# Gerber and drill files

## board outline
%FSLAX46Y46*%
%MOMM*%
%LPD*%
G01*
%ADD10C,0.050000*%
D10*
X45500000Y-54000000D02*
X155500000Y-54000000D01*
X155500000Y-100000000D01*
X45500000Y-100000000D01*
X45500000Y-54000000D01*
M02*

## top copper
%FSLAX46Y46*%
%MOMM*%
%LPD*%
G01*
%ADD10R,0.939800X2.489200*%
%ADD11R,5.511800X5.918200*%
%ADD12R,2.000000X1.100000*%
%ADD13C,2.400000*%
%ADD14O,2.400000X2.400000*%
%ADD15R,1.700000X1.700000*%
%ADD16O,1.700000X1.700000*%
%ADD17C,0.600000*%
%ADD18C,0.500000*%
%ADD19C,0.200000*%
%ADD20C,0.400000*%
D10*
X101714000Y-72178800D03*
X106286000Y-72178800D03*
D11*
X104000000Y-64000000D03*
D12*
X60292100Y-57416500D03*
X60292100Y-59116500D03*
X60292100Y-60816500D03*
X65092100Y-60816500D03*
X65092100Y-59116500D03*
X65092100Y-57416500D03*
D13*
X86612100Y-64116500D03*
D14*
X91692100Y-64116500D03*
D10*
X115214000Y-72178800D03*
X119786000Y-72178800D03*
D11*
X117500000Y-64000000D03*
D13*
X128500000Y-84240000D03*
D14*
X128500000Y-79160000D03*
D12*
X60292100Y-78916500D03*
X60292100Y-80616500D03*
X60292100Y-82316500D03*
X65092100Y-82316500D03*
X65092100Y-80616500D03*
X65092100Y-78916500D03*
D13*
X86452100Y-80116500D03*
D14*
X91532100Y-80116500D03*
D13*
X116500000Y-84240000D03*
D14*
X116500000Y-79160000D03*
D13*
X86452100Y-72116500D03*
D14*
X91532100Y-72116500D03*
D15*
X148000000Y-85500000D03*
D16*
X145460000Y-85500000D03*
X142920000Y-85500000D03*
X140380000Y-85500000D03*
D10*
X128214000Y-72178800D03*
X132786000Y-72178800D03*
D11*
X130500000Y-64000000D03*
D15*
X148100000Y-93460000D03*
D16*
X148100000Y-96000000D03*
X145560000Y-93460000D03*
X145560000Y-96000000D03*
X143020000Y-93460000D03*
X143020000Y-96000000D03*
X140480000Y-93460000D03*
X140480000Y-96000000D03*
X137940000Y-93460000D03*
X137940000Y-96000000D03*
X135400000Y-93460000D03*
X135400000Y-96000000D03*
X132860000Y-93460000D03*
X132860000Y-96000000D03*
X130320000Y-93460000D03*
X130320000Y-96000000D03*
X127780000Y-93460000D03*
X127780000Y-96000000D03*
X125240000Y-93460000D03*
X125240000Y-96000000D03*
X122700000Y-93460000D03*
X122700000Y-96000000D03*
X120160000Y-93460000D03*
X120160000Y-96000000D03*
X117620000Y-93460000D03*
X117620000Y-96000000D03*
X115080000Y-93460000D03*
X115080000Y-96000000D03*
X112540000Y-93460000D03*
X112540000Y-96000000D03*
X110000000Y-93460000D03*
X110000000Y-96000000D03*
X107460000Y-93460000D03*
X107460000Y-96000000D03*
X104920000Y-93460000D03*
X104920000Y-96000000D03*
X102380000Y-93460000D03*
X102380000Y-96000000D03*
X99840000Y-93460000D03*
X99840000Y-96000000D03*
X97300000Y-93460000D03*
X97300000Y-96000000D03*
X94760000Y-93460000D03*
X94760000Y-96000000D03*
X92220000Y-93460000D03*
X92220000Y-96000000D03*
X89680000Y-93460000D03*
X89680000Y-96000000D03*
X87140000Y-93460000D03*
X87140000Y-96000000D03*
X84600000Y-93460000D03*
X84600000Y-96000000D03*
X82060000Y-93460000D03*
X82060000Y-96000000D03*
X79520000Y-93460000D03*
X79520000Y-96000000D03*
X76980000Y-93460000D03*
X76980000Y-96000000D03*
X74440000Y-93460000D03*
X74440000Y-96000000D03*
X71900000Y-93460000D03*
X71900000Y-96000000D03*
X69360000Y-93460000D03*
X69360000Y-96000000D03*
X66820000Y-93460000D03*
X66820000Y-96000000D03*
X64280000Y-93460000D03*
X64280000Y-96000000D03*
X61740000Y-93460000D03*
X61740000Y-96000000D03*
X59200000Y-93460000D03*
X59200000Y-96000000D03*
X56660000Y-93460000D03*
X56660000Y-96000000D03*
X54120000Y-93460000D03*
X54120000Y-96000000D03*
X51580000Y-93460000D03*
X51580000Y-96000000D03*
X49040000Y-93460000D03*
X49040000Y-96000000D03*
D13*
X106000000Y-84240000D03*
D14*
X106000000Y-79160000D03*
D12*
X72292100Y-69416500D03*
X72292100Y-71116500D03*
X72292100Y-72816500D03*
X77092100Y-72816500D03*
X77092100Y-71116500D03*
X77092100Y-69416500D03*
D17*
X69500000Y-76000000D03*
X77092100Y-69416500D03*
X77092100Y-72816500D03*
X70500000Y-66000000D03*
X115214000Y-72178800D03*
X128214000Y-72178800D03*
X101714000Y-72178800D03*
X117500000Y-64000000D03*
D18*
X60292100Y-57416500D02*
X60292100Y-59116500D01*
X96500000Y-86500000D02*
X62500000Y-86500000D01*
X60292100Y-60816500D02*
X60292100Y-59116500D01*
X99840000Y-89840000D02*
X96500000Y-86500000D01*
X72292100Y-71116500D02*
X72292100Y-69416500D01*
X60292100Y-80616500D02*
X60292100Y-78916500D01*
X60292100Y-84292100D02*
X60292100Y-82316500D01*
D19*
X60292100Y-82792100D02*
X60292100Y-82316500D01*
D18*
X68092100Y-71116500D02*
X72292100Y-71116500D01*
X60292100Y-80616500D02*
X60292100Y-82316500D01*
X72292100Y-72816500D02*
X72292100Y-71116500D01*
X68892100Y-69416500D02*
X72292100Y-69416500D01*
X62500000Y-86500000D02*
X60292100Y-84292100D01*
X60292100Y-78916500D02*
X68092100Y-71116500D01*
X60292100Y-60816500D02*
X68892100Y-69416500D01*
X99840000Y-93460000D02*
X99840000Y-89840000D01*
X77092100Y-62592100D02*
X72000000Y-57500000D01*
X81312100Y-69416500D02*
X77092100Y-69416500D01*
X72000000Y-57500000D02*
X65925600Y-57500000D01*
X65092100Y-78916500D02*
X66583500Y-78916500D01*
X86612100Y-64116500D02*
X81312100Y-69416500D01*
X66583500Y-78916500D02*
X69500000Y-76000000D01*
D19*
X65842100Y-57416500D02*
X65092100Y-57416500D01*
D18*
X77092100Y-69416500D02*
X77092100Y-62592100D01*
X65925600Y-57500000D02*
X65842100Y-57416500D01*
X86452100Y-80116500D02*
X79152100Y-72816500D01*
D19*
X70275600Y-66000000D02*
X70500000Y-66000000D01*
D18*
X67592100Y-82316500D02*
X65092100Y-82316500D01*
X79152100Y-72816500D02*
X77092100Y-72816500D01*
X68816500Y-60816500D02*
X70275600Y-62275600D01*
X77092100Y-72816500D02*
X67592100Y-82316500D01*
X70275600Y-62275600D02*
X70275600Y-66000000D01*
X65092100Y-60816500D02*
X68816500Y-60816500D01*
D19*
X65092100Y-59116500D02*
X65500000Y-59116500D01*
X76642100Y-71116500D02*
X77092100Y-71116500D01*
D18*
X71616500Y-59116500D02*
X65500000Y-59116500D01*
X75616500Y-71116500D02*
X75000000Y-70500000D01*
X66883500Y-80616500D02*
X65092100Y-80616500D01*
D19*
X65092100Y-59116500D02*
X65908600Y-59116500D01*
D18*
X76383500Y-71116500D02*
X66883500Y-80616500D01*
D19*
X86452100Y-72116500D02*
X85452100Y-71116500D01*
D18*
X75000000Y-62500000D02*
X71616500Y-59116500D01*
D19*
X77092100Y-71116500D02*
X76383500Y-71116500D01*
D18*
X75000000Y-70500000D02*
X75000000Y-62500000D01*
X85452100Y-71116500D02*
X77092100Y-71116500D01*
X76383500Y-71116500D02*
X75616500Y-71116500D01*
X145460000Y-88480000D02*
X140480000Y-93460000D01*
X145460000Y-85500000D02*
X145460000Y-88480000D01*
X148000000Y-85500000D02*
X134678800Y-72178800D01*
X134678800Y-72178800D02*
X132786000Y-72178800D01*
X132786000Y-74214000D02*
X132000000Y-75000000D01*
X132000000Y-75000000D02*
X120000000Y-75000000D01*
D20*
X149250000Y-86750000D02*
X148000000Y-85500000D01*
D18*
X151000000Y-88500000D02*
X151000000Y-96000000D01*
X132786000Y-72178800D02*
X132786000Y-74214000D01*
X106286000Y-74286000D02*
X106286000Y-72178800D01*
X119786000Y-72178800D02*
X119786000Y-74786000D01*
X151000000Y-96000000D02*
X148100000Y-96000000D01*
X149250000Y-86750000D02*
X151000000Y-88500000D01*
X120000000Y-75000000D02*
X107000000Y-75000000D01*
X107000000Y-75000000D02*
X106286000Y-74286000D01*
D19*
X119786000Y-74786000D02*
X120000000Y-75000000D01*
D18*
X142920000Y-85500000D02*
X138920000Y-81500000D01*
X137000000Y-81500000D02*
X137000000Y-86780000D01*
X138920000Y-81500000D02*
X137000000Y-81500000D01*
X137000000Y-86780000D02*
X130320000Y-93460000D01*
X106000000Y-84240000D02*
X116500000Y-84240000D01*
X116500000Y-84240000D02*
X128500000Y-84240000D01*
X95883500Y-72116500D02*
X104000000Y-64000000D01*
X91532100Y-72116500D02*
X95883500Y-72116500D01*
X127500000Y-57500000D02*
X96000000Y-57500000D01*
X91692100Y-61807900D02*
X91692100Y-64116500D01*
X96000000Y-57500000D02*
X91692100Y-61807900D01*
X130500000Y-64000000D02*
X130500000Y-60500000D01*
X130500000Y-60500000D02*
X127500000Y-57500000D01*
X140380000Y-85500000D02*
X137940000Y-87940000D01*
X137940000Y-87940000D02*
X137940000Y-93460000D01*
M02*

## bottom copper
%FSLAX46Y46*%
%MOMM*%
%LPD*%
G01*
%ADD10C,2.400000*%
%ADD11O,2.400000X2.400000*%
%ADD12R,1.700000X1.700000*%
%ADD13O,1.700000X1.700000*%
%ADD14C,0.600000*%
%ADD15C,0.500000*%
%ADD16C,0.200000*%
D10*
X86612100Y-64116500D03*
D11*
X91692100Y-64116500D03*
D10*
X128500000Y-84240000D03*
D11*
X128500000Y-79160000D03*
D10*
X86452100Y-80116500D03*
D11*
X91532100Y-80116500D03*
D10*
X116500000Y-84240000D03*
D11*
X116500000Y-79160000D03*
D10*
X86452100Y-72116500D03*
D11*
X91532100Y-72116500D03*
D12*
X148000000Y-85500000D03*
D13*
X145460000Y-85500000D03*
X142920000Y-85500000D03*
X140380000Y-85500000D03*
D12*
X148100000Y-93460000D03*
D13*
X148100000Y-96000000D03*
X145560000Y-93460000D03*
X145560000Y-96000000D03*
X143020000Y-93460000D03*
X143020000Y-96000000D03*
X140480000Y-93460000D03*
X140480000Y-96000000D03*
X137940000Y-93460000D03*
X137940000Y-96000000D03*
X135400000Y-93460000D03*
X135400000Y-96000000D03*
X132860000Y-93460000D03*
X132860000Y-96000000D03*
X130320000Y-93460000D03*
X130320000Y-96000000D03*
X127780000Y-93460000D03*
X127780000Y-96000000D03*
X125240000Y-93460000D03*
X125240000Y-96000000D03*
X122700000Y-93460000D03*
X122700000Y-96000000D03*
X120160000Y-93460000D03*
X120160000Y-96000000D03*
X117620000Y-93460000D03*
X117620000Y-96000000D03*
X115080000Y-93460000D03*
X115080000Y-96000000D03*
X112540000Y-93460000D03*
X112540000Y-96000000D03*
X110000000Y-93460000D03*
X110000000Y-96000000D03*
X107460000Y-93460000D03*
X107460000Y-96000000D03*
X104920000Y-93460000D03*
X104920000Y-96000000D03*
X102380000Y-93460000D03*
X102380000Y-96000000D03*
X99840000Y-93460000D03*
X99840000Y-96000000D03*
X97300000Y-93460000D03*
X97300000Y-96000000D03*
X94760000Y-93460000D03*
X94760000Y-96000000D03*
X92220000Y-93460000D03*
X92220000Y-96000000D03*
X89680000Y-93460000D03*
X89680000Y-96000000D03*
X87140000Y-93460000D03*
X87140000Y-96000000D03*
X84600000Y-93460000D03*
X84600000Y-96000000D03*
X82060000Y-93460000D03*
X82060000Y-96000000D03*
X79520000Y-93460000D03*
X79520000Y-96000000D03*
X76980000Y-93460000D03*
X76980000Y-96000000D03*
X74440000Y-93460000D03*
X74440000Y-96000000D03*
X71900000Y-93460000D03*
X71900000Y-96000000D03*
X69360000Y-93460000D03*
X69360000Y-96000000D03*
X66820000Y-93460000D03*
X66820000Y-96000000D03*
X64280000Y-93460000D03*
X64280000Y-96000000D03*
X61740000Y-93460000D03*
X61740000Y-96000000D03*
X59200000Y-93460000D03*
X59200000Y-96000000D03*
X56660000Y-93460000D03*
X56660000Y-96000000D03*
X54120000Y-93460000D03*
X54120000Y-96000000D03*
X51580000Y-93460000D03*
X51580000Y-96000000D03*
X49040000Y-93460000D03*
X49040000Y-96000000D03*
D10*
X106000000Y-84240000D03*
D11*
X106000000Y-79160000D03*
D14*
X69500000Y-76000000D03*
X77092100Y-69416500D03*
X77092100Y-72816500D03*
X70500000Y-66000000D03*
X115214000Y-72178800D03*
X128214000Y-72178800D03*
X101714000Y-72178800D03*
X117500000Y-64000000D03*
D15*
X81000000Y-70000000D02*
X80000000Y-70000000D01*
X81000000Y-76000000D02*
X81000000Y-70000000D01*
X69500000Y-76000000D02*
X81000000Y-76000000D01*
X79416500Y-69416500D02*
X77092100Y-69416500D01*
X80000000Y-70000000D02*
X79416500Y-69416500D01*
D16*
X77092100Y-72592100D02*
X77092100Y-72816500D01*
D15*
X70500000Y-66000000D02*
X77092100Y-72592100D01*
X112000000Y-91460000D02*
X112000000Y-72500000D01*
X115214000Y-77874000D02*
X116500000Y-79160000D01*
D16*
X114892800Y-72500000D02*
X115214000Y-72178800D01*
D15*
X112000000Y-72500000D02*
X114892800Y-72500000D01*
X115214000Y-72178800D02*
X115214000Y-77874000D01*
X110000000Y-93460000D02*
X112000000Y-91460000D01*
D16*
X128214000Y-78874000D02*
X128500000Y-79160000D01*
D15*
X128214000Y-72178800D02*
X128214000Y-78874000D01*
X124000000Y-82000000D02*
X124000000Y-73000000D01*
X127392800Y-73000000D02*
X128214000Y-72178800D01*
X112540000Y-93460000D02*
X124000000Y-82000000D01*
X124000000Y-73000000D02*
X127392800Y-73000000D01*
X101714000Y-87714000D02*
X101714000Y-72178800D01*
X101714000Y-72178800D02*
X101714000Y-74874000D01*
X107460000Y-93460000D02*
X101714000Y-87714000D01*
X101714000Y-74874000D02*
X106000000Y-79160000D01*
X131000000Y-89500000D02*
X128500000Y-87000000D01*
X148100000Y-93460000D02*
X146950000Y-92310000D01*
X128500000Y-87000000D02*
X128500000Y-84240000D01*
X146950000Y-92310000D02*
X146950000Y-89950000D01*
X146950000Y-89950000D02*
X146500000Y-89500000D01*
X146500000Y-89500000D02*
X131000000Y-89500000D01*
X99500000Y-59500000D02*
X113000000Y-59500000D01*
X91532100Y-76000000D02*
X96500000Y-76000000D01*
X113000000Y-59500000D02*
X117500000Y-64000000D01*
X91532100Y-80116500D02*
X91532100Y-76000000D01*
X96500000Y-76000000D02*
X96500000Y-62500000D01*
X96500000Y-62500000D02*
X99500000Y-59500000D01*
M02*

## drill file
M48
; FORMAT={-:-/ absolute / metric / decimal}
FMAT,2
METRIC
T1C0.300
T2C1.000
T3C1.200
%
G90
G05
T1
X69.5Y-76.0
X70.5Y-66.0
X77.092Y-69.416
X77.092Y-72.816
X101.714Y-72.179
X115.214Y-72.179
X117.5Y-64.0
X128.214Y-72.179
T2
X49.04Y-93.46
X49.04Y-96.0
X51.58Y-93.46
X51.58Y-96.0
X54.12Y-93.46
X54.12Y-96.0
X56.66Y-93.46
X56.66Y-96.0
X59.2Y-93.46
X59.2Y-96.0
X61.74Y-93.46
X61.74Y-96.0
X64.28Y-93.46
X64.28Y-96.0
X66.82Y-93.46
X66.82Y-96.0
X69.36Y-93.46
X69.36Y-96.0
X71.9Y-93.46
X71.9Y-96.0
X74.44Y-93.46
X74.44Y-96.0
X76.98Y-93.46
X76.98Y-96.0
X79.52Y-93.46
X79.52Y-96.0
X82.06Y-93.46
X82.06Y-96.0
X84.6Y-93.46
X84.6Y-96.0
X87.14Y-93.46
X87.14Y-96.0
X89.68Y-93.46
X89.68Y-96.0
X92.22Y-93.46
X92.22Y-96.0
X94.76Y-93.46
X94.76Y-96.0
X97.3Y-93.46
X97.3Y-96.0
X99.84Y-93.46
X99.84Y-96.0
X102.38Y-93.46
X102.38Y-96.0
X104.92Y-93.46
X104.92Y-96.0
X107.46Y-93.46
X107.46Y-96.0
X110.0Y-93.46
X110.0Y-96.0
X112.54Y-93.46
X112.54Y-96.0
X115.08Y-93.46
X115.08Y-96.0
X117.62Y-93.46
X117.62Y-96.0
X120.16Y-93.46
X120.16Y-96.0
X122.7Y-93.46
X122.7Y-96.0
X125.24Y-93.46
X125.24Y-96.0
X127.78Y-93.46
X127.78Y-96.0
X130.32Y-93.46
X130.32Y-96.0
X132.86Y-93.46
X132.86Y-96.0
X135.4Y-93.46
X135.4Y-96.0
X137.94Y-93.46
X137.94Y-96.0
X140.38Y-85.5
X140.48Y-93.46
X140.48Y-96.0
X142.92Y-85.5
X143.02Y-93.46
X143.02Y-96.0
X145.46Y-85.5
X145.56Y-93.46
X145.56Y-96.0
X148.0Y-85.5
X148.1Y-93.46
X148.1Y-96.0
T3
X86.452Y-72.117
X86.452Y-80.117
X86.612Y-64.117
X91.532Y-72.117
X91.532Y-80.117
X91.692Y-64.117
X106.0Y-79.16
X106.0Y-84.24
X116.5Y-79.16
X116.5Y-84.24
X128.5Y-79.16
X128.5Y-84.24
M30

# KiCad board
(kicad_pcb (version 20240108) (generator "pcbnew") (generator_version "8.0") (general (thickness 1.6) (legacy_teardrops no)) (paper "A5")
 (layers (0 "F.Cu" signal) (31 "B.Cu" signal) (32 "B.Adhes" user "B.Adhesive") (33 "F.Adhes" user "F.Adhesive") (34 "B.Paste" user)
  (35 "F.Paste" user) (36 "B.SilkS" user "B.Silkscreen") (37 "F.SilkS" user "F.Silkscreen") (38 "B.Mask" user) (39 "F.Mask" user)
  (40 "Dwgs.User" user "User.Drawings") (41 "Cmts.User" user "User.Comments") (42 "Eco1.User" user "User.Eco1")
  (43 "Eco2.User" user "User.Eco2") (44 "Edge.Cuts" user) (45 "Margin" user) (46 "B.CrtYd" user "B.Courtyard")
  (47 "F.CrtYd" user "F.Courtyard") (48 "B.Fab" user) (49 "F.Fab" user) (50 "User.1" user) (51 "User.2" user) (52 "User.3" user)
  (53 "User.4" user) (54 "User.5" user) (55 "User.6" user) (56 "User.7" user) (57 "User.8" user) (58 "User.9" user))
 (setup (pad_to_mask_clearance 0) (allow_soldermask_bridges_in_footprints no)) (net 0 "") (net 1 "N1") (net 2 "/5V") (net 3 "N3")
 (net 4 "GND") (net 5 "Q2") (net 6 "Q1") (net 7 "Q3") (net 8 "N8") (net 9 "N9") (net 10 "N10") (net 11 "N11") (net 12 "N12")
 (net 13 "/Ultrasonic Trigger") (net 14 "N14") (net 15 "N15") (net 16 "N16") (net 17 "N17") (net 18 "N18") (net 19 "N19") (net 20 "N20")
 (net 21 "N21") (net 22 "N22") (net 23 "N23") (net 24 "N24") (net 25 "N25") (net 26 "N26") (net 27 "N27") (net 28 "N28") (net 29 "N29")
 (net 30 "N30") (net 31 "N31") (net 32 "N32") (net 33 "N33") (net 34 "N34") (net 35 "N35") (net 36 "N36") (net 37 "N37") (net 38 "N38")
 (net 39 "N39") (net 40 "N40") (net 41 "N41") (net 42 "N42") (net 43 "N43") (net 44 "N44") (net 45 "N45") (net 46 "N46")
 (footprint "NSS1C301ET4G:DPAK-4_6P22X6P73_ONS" (layer "F.Cu") (at 104 65.7653)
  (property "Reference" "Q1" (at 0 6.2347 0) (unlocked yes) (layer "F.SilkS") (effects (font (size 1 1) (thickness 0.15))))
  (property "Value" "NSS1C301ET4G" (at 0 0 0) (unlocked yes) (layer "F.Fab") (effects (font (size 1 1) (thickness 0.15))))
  (pad "1" smd rect (at -2.286 6.4135) (size 0.9398 2.4892) (layers "F.Cu" "F.Paste" "F.Mask") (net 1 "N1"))
  (pad "2" smd rect (at 2.286 6.4135) (size 0.9398 2.4892) (layers "F.Cu" "F.Paste" "F.Mask") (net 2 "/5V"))
  (pad "3" smd rect (at 0 -1.7653) (size 5.5118 5.9182) (layers "F.Cu" "F.Paste" "F.Mask") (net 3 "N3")))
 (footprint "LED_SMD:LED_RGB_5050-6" (layer "F.Cu") (at 62.6921 59.1165)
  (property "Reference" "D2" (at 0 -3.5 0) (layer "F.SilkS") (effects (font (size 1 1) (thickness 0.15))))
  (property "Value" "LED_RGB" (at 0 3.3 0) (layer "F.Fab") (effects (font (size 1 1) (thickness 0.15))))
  (pad "1" smd rect (at -2.4 -1.7 90) (size 1.1 2) (layers "F.Cu" "F.Paste" "F.Mask") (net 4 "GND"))
  (pad "2" smd rect (at -2.4 0 90) (size 1.1 2) (layers "F.Cu" "F.Paste" "F.Mask") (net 4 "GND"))
  (pad "3" smd rect (at -2.4 1.7 90) (size 1.1 2) (layers "F.Cu" "F.Paste" "F.Mask") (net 4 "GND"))
  (pad "4" smd rect (at 2.4 1.7 90) (size 1.1 2) (layers "F.Cu" "F.Paste" "F.Mask") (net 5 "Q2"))
  (pad "5" smd rect (at 2.4 0 90) (size 1.1 2) (layers "F.Cu" "F.Paste" "F.Mask") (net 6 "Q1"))
  (pad "6" smd rect (at 2.4 -1.7 90) (size 1.1 2) (layers "F.Cu" "F.Paste" "F.Mask") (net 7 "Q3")))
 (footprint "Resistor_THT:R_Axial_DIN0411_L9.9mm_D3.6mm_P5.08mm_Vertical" (layer "F.Cu") (at 86.6121 64.1165)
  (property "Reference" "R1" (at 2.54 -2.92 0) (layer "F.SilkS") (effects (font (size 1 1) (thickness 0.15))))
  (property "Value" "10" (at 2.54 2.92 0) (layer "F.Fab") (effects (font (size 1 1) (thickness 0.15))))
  (pad "1" thru_hole circle (at 0 0) (size 2.4 2.4) (drill 1.2) (layers "*.Cu" "*.Mask") (remove_unused_layers no) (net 7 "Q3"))
  (pad "2" thru_hole oval (at 5.08 0) (size 2.4 2.4) (drill 1.2) (layers "*.Cu" "*.Mask") (remove_unused_layers no) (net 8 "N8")))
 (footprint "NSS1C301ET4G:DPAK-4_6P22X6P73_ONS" (layer "F.Cu") (at 117.5 65.7653)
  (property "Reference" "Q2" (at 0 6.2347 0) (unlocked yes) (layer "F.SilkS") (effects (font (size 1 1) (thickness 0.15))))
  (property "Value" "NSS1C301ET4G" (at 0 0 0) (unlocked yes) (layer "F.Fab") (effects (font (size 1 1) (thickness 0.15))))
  (pad "1" smd rect (at -2.286 6.4135) (size 0.9398 2.4892) (layers "F.Cu" "F.Paste" "F.Mask") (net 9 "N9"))
  (pad "2" smd rect (at 2.286 6.4135) (size 0.9398 2.4892) (layers "F.Cu" "F.Paste" "F.Mask") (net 2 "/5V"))
  (pad "3" smd rect (at 0 -1.7653) (size 5.5118 5.9182) (layers "F.Cu" "F.Paste" "F.Mask") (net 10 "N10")))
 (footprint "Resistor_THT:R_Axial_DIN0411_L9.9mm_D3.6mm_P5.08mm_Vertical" (layer "F.Cu") (at 128.5 84.24 90)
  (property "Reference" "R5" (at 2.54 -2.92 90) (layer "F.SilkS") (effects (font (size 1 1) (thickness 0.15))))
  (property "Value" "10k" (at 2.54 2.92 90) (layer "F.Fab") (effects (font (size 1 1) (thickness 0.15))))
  (pad "1" thru_hole circle (at 0 0 90) (size 2.4 2.4) (drill 1.2) (layers "*.Cu" "*.Mask") (remove_unused_layers no) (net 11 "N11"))
  (pad "2" thru_hole oval (at 5.08 0 90) (size 2.4 2.4) (drill 1.2) (layers "*.Cu" "*.Mask") (remove_unused_layers no) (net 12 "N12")))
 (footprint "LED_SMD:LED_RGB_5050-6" (layer "F.Cu") (at 62.6921 80.6165)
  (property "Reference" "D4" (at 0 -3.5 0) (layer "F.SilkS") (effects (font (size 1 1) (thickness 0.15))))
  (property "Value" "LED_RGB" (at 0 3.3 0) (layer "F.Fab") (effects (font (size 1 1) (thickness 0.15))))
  (pad "1" smd rect (at -2.4 -1.7 90) (size 1.1 2) (layers "F.Cu" "F.Paste" "F.Mask") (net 4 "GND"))
  (pad "2" smd rect (at -2.4 0 90) (size 1.1 2) (layers "F.Cu" "F.Paste" "F.Mask") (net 4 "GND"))
  (pad "3" smd rect (at -2.4 1.7 90) (size 1.1 2) (layers "F.Cu" "F.Paste" "F.Mask") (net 4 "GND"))
  (pad "4" smd rect (at 2.4 1.7 90) (size 1.1 2) (layers "F.Cu" "F.Paste" "F.Mask") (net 5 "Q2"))
  (pad "5" smd rect (at 2.4 0 90) (size 1.1 2) (layers "F.Cu" "F.Paste" "F.Mask") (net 6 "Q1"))
  (pad "6" smd rect (at 2.4 -1.7 90) (size 1.1 2) (layers "F.Cu" "F.Paste" "F.Mask") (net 7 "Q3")))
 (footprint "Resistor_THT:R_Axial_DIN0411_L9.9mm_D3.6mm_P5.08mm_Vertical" (layer "F.Cu") (at 86.4521 80.1165)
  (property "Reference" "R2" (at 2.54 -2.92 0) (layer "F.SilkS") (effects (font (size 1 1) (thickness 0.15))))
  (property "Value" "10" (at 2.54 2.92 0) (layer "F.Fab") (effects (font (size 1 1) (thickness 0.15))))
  (pad "1" thru_hole circle (at 0 0) (size 2.4 2.4) (drill 1.2) (layers "*.Cu" "*.Mask") (remove_unused_layers no) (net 5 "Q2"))
  (pad "2" thru_hole oval (at 5.08 0) (size 2.4 2.4) (drill 1.2) (layers "*.Cu" "*.Mask") (remove_unused_layers no) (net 10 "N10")))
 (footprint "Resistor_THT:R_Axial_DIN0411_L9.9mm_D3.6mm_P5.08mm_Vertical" (layer "F.Cu") (at 116.5 84.24 90)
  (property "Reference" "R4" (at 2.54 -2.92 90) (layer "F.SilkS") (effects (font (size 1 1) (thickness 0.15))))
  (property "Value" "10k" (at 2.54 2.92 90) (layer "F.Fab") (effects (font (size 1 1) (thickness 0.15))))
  (pad "1" thru_hole circle (at 0 0 90) (size 2.4 2.4) (drill 1.2) (layers "*.Cu" "*.Mask") (remove_unused_layers no) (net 11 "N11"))
  (pad "2" thru_hole oval (at 5.08 0 90) (size 2.4 2.4) (drill 1.2) (layers "*.Cu" "*.Mask") (remove_unused_layers no) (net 9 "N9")))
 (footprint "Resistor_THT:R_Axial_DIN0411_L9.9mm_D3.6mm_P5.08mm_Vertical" (layer "F.Cu") (at 86.4521 72.1165)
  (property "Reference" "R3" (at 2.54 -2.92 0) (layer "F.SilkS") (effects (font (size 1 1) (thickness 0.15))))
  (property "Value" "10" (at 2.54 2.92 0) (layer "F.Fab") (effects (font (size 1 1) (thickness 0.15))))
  (pad "1" thru_hole circle (at 0 0) (size 2.4 2.4) (drill 1.2) (layers "*.Cu" "*.Mask") (remove_unused_layers no) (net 6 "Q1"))
  (pad "2" thru_hole oval (at 5.08 0) (size 2.4 2.4) (drill 1.2) (layers "*.Cu" "*.Mask") (remove_unused_layers no) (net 3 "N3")))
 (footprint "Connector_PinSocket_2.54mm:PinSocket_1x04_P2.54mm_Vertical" (layer "F.Cu") (at 148 85.5 -90)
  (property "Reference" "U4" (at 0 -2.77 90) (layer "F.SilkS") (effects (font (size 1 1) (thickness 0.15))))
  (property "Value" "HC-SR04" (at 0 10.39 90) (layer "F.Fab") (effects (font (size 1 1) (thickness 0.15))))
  (pad "1" thru_hole rect (at 0 0 270) (size 1.7 1.7) (drill 1) (layers "*.Cu" "*.Mask") (remove_unused_layers no) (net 2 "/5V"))
  (pad "2" thru_hole oval (at 0 2.54 270) (size 1.7 1.7) (drill 1) (layers "*.Cu" "*.Mask") (remove_unused_layers no)
   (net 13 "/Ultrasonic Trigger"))
  (pad "3" thru_hole oval (at 0 5.08 270) (size 1.7 1.7) (drill 1) (layers "*.Cu" "*.Mask") (remove_unused_layers no) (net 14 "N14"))
  (pad "4" thru_hole oval (at 0 7.62 270) (size 1.7 1.7) (drill 1) (layers "*.Cu" "*.Mask") (remove_unused_layers no) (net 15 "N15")))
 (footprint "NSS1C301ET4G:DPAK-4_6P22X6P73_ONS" (layer "F.Cu") (at 130.5 65.7653)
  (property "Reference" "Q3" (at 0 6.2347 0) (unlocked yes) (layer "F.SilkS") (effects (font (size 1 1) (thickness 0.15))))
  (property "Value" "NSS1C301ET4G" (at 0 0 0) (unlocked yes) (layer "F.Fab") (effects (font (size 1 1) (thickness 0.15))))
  (pad "1" smd rect (at -2.286 6.4135) (size 0.9398 2.4892) (layers "F.Cu" "F.Paste" "F.Mask") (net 12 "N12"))
  (pad "2" smd rect (at 2.286 6.4135) (size 0.9398 2.4892) (layers "F.Cu" "F.Paste" "F.Mask") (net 2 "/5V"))
  (pad "3" smd rect (at 0 -1.7653) (size 5.5118 5.9182) (layers "F.Cu" "F.Paste" "F.Mask") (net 8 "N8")))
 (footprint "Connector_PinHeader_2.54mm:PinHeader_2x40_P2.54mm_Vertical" (layer "F.Cu") (at 148.1 93.46 -90)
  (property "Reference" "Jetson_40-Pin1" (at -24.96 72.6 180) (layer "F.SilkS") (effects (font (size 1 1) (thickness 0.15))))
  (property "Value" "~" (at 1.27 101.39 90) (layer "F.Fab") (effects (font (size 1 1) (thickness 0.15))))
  (pad "1" thru_hole rect (at 0 0 270) (size 1.7 1.7) (drill 1) (layers "*.Cu" "*.Mask") (remove_unused_layers no) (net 11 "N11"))
  (pad "2" thru_hole oval (at 2.54 0 270) (size 1.7 1.7) (drill 1) (layers "*.Cu" "*.Mask") (remove_unused_layers no) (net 2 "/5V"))
  (pad "3" thru_hole oval (at 0 2.54 270) (size 1.7 1.7) (drill 1) (layers "*.Cu" "*.Mask") (remove_unused_layers no) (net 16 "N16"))
  (pad "4" thru_hole oval (at 2.54 2.54 270) (size 1.7 1.7) (drill 1) (layers "*.Cu" "*.Mask") (remove_unused_layers no) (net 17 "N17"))
  (pad "5" thru_hole oval (at 0 5.08 270) (size 1.7 1.7) (drill 1) (layers "*.Cu" "*.Mask") (remove_unused_layers no) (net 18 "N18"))
  (pad "6" thru_hole oval (at 2.54 5.08 270) (size 1.7 1.7) (drill 1) (layers "*.Cu" "*.Mask") (remove_unused_layers no) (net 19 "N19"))
  (pad "7" thru_hole oval (at 0 7.62 270) (size 1.7 1.7) (drill 1) (layers "*.Cu" "*.Mask") (remove_unused_layers no)
   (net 13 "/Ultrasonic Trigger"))
  (pad "8" thru_hole oval (at 2.54 7.62 270) (size 1.7 1.7) (drill 1) (layers "*.Cu" "*.Mask") (remove_unused_layers no) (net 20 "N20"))
  (pad "9" thru_hole oval (at 0 10.16 270) (size 1.7 1.7) (drill 1) (layers "*.Cu" "*.Mask") (remove_unused_layers no) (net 15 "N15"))
  (pad "10" thru_hole oval (at 2.54 10.16 270) (size 1.7 1.7) (drill 1) (layers "*.Cu" "*.Mask") (remove_unused_layers no) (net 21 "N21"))
  (pad "11" thru_hole oval (at 0 12.7 270) (size 1.7 1.7) (drill 1) (layers "*.Cu" "*.Mask") (remove_unused_layers no) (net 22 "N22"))
  (pad "12" thru_hole oval (at 2.54 12.7 270) (size 1.7 1.7) (drill 1) (layers "*.Cu" "*.Mask") (remove_unused_layers no) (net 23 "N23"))
  (pad "13" thru_hole oval (at 0 15.24 270) (size 1.7 1.7) (drill 1) (layers "*.Cu" "*.Mask") (remove_unused_layers no) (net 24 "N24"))
  (pad "14" thru_hole oval (at 2.54 15.24 270) (size 1.7 1.7) (drill 1) (layers "*.Cu" "*.Mask") (remove_unused_layers no) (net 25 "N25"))
  (pad "15" thru_hole oval (at 0 17.78 270) (size 1.7 1.7) (drill 1) (layers "*.Cu" "*.Mask") (remove_unused_layers no) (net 14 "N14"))
  (pad "16" thru_hole oval (at 2.54 17.78 270) (size 1.7 1.7) (drill 1) (layers "*.Cu" "*.Mask") (remove_unused_layers no) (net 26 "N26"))
  (pad "17" thru_hole oval (at 0 20.32 270) (size 1.7 1.7) (drill 1) (layers "*.Cu" "*.Mask") (remove_unused_layers no) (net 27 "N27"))
  (pad "18" thru_hole oval (at 2.54 20.32 270) (size 1.7 1.7) (drill 1) (layers "*.Cu" "*.Mask") (remove_unused_layers no) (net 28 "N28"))
  (pad "19" thru_hole oval (at 0 22.86 270) (size 1.7 1.7) (drill 1) (layers "*.Cu" "*.Mask") (remove_unused_layers no) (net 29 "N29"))
  (pad "20" thru_hole oval (at 2.54 22.86 270) (size 1.7 1.7) (drill 1) (layers "*.Cu" "*.Mask") (remove_unused_layers no) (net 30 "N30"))
  (pad "21" thru_hole oval (at 0 25.4 270) (size 1.7 1.7) (drill 1) (layers "*.Cu" "*.Mask") (remove_unused_layers no) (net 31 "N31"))
  (pad "22" thru_hole oval (at 2.54 25.4 270) (size 1.7 1.7) (drill 1) (layers "*.Cu" "*.Mask") (remove_unused_layers no) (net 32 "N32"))
  (pad "23" thru_hole oval (at 0 27.94 270) (size 1.7 1.7) (drill 1) (layers "*.Cu" "*.Mask") (remove_unused_layers no) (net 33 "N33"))
  (pad "24" thru_hole oval (at 2.54 27.94 270) (size 1.7 1.7) (drill 1) (layers "*.Cu" "*.Mask") (remove_unused_layers no) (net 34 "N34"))
  (pad "25" thru_hole oval (at 0 30.48 270) (size 1.7 1.7) (drill 1) (layers "*.Cu" "*.Mask") (remove_unused_layers no) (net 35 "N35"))
  (pad "26" thru_hole oval (at 2.54 30.48 270) (size 1.7 1.7) (drill 1) (layers "*.Cu" "*.Mask") (remove_unused_layers no) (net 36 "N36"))
  (pad "27" thru_hole oval (at 0 33.02 270) (size 1.7 1.7) (drill 1) (layers "*.Cu" "*.Mask") (remove_unused_layers no) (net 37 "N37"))
  (pad "28" thru_hole oval (at 2.54 33.02 270) (size 1.7 1.7) (drill 1) (layers "*.Cu" "*.Mask") (remove_unused_layers no) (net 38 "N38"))
  (pad "29" thru_hole oval (at 0 35.56 270) (size 1.7 1.7) (drill 1) (layers "*.Cu" "*.Mask") (remove_unused_layers no) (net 12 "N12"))
  (pad "30" thru_hole oval (at 2.54 35.56 270) (size 1.7 1.7) (drill 1) (layers "*.Cu" "*.Mask") (remove_unused_layers no) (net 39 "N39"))
  (pad "31" thru_hole oval (at 0 38.1 270) (size 1.7 1.7) (drill 1) (layers "*.Cu" "*.Mask") (remove_unused_layers no) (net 9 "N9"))
  (pad "32" thru_hole oval (at 2.54 38.1 270) (size 1.7 1.7) (drill 1) (layers "*.Cu" "*.Mask") (remove_unused_layers no) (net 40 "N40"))
  (pad "33" thru_hole oval (at 0 40.64 270) (size 1.7 1.7) (drill 1) (layers "*.Cu" "*.Mask") (remove_unused_layers no) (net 1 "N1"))
  (pad "34" thru_hole oval (at 2.54 40.64 270) (size 1.7 1.7) (drill 1) (layers "*.Cu" "*.Mask") (remove_unused_layers no) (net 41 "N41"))
  (pad "35" thru_hole oval (at 0 43.18 270) (size 1.7 1.7) (drill 1) (layers "*.Cu" "*.Mask") (remove_unused_layers no) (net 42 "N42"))
  (pad "36" thru_hole oval (at 2.54 43.18 270) (size 1.7 1.7) (drill 1) (layers "*.Cu" "*.Mask") (remove_unused_layers no) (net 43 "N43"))
  (pad "37" thru_hole oval (at 0 45.72 270) (size 1.7 1.7) (drill 1) (layers "*.Cu" "*.Mask") (remove_unused_layers no) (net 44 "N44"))
  (pad "38" thru_hole oval (at 2.54 45.72 270) (size 1.7 1.7) (drill 1) (layers "*.Cu" "*.Mask") (remove_unused_layers no) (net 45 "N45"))
  (pad "39" thru_hole oval (at 0 48.26 270) (size 1.7 1.7) (drill 1) (layers "*.Cu" "*.Mask") (remove_unused_layers no) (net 4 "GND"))
  (pad "40" thru_hole oval (at 2.54 48.26 270) (size 1.7 1.7) (drill 1) (layers "*.Cu" "*.Mask") (remove_unused_layers no) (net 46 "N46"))
  (pad "41" thru_hole oval (at 0 50.8 270) (size 1.7 1.7) (drill 1) (layers "*.Cu" "*.Mask") (remove_unused_layers no))
  (pad "42" thru_hole oval (at 2.54 50.8 270) (size 1.7 1.7) (drill 1) (layers "*.Cu" "*.Mask") (remove_unused_layers no))
  (pad "43" thru_hole oval (at 0 53.34 270) (size 1.7 1.7) (drill 1) (layers "*.Cu" "*.Mask") (remove_unused_layers no))
  (pad "44" thru_hole oval (at 2.54 53.34 270) (size 1.7 1.7) (drill 1) (layers "*.Cu" "*.Mask") (remove_unused_layers no))
  (pad "45" thru_hole oval (at 0 55.88 270) (size 1.7 1.7) (drill 1) (layers "*.Cu" "*.Mask") (remove_unused_layers no))
  (pad "46" thru_hole oval (at 2.54 55.88 270) (size 1.7 1.7) (drill 1) (layers "*.Cu" "*.Mask") (remove_unused_layers no))
  (pad "47" thru_hole oval (at 0 58.42 270) (size 1.7 1.7) (drill 1) (layers "*.Cu" "*.Mask") (remove_unused_layers no))
  (pad "48" thru_hole oval (at 2.54 58.42 270) (size 1.7 1.7) (drill 1) (layers "*.Cu" "*.Mask") (remove_unused_layers no))
  (pad "49" thru_hole oval (at 0 60.96 270) (size 1.7 1.7) (drill 1) (layers "*.Cu" "*.Mask") (remove_unused_layers no))
  (pad "50" thru_hole oval (at 2.54 60.96 270) (size 1.7 1.7) (drill 1) (layers "*.Cu" "*.Mask") (remove_unused_layers no))
  (pad "51" thru_hole oval (at 0 63.5 270) (size 1.7 1.7) (drill 1) (layers "*.Cu" "*.Mask") (remove_unused_layers no))
  (pad "52" thru_hole oval (at 2.54 63.5 270) (size 1.7 1.7) (drill 1) (layers "*.Cu" "*.Mask") (remove_unused_layers no))
  (pad "53" thru_hole oval (at 0 66.04 270) (size 1.7 1.7) (drill 1) (layers "*.Cu" "*.Mask") (remove_unused_layers no))
  (pad "54" thru_hole oval (at 2.54 66.04 270) (size 1.7 1.7) (drill 1) (layers "*.Cu" "*.Mask") (remove_unused_layers no))
  (pad "55" thru_hole oval (at 0 68.58 270) (size 1.7 1.7) (drill 1) (layers "*.Cu" "*.Mask") (remove_unused_layers no))
  (pad "56" thru_hole oval (at 2.54 68.58 270) (size 1.7 1.7) (drill 1) (layers "*.Cu" "*.Mask") (remove_unused_layers no))
  (pad "57" thru_hole oval (at 0 71.12 270) (size 1.7 1.7) (drill 1) (layers "*.Cu" "*.Mask") (remove_unused_layers no))
  (pad "58" thru_hole oval (at 2.54 71.12 270) (size 1.7 1.7) (drill 1) (layers "*.Cu" "*.Mask") (remove_unused_layers no))
  (pad "59" thru_hole oval (at 0 73.66 270) (size 1.7 1.7) (drill 1) (layers "*.Cu" "*.Mask") (remove_unused_layers no))
  (pad "60" thru_hole oval (at 2.54 73.66 270) (size 1.7 1.7) (drill 1) (layers "*.Cu" "*.Mask") (remove_unused_layers no))
  (pad "61" thru_hole oval (at 0 76.2 270) (size 1.7 1.7) (drill 1) (layers "*.Cu" "*.Mask") (remove_unused_layers no))
  (pad "62" thru_hole oval (at 2.54 76.2 270) (size 1.7 1.7) (drill 1) (layers "*.Cu" "*.Mask") (remove_unused_layers no))
  (pad "63" thru_hole oval (at 0 78.74 270) (size 1.7 1.7) (drill 1) (layers "*.Cu" "*.Mask") (remove_unused_layers no))
  (pad "64" thru_hole oval (at 2.54 78.74 270) (size 1.7 1.7) (drill 1) (layers "*.Cu" "*.Mask") (remove_unused_layers no))
  (pad "65" thru_hole oval (at 0 81.28 270) (size 1.7 1.7) (drill 1) (layers "*.Cu" "*.Mask") (remove_unused_layers no))
  (pad "66" thru_hole oval (at 2.54 81.28 270) (size 1.7 1.7) (drill 1) (layers "*.Cu" "*.Mask") (remove_unused_layers no))
  (pad "67" thru_hole oval (at 0 83.82 270) (size 1.7 1.7) (drill 1) (layers "*.Cu" "*.Mask") (remove_unused_layers no))
  (pad "68" thru_hole oval (at 2.54 83.82 270) (size 1.7 1.7) (drill 1) (layers "*.Cu" "*.Mask") (remove_unused_layers no))
  (pad "69" thru_hole oval (at 0 86.36 270) (size 1.7 1.7) (drill 1) (layers "*.Cu" "*.Mask") (remove_unused_layers no))
  (pad "70" thru_hole oval (at 2.54 86.36 270) (size 1.7 1.7) (drill 1) (layers "*.Cu" "*.Mask") (remove_unused_layers no))
  (pad "71" thru_hole oval (at 0 88.9 270) (size 1.7 1.7) (drill 1) (layers "*.Cu" "*.Mask") (remove_unused_layers no))
  (pad "72" thru_hole oval (at 2.54 88.9 270) (size 1.7 1.7) (drill 1) (layers "*.Cu" "*.Mask") (remove_unused_layers no))
  (pad "73" thru_hole oval (at 0 91.44 270) (size 1.7 1.7) (drill 1) (layers "*.Cu" "*.Mask") (remove_unused_layers no))
  (pad "74" thru_hole oval (at 2.54 91.44 270) (size 1.7 1.7) (drill 1) (layers "*.Cu" "*.Mask") (remove_unused_layers no))
  (pad "75" thru_hole oval (at 0 93.98 270) (size 1.7 1.7) (drill 1) (layers "*.Cu" "*.Mask") (remove_unused_layers no))
  (pad "76" thru_hole oval (at 2.54 93.98 270) (size 1.7 1.7) (drill 1) (layers "*.Cu" "*.Mask") (remove_unused_layers no))
  (pad "77" thru_hole oval (at 0 96.52 270) (size 1.7 1.7) (drill 1) (layers "*.Cu" "*.Mask") (remove_unused_layers no))
  (pad "78" thru_hole oval (at 2.54 96.52 270) (size 1.7 1.7) (drill 1) (layers "*.Cu" "*.Mask") (remove_unused_layers no))
  (pad "79" thru_hole oval (at 0 99.06 270) (size 1.7 1.7) (drill 1) (layers "*.Cu" "*.Mask") (remove_unused_layers no))
  (pad "80" thru_hole oval (at 2.54 99.06 270) (size 1.7 1.7) (drill 1) (layers "*.Cu" "*.Mask") (remove_unused_layers no)))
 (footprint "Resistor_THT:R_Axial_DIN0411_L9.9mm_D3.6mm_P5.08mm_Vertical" (layer "F.Cu") (at 106 84.24 90)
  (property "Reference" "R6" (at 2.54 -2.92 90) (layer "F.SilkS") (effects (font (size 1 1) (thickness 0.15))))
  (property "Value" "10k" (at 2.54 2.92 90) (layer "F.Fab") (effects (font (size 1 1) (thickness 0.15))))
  (pad "1" thru_hole circle (at 0 0 90) (size 2.4 2.4) (drill 1.2) (layers "*.Cu" "*.Mask") (remove_unused_layers no) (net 11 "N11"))
  (pad "2" thru_hole oval (at 5.08 0 90) (size 2.4 2.4) (drill 1.2) (layers "*.Cu" "*.Mask") (remove_unused_layers no) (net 1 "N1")))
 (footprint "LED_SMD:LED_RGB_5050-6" (layer "F.Cu") (at 74.6921 71.1165)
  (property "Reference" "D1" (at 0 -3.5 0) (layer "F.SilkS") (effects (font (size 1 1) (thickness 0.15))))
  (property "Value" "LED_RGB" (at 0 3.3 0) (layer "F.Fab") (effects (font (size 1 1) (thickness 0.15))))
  (pad "1" smd rect (at -2.4 -1.7 90) (size 1.1 2) (layers "F.Cu" "F.Paste" "F.Mask") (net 4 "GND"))
  (pad "2" smd rect (at -2.4 0 90) (size 1.1 2) (layers "F.Cu" "F.Paste" "F.Mask") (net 4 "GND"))
  (pad "3" smd rect (at -2.4 1.7 90) (size 1.1 2) (layers "F.Cu" "F.Paste" "F.Mask") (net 4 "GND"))
  (pad "4" smd rect (at 2.4 1.7 90) (size 1.1 2) (layers "F.Cu" "F.Paste" "F.Mask") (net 5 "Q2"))
  (pad "5" smd rect (at 2.4 0 90) (size 1.1 2) (layers "F.Cu" "F.Paste" "F.Mask") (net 6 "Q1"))
  (pad "6" smd rect (at 2.4 -1.7 90) (size 1.1 2) (layers "F.Cu" "F.Paste" "F.Mask") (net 7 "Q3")))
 (gr_rect (start 45.5 54) (end 155.5 100) (stroke (width 0.05) (type default)) (fill none) (layer "Edge.Cuts"))
 (segment (start 60.2921 57.4165) (end 60.2921 59.1165) (width 0.5) (layer "F.Cu") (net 4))
 (segment (start 96.5 86.5) (end 62.5 86.5) (width 0.5) (layer "F.Cu") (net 4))
 (segment (start 60.2921 60.8165) (end 60.2921 59.1165) (width 0.5) (layer "F.Cu") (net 4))
 (segment (start 99.84 89.84) (end 96.5 86.5) (width 0.5) (layer "F.Cu") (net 4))
 (segment (start 72.2921 71.1165) (end 72.2921 69.4165) (width 0.5) (layer "F.Cu") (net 4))
 (segment (start 60.2921 80.6165) (end 60.2921 78.9165) (width 0.5) (layer "F.Cu") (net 4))
 (segment (start 60.2921 84.2921) (end 60.2921 82.3165) (width 0.5) (layer "F.Cu") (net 4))
 (segment (start 60.2921 82.7921) (end 60.2921 82.3165) (width 0.2) (layer "F.Cu") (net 4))
 (segment (start 68.0921 71.1165) (end 72.2921 71.1165) (width 0.5) (layer "F.Cu") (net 4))
 (segment (start 60.2921 80.6165) (end 60.2921 82.3165) (width 0.5) (layer "F.Cu") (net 4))
 (segment (start 72.2921 72.8165) (end 72.2921 71.1165) (width 0.5) (layer "F.Cu") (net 4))
 (segment (start 68.8921 69.4165) (end 72.2921 69.4165) (width 0.5) (layer "F.Cu") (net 4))
 (segment (start 62.5 86.5) (end 60.2921 84.2921) (width 0.5) (layer "F.Cu") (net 4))
 (segment (start 60.2921 78.9165) (end 68.0921 71.1165) (width 0.5) (layer "F.Cu") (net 4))
 (segment (start 60.2921 60.8165) (end 68.8921 69.4165) (width 0.5) (layer "F.Cu") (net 4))
 (segment (start 99.84 93.46) (end 99.84 89.84) (width 0.5) (layer "F.Cu") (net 4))
 (segment (start 77.0921 62.5921) (end 72 57.5) (width 0.5) (layer "F.Cu") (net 7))
 (segment (start 81.3121 69.4165) (end 77.0921 69.4165) (width 0.5) (layer "F.Cu") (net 7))
 (segment (start 72 57.5) (end 65.9256 57.5) (width 0.5) (layer "F.Cu") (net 7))
 (segment (start 65.0921 78.9165) (end 66.5835 78.9165) (width 0.5) (layer "F.Cu") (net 7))
 (segment (start 86.6121 64.1165) (end 81.3121 69.4165) (width 0.5) (layer "F.Cu") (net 7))
 (segment (start 66.5835 78.9165) (end 69.5 76) (width 0.5) (layer "F.Cu") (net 7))
 (segment (start 65.8421 57.4165) (end 65.0921 57.4165) (width 0.2) (layer "F.Cu") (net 7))
 (segment (start 77.0921 69.4165) (end 77.0921 62.5921) (width 0.5) (layer "F.Cu") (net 7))
 (segment (start 65.9256 57.5) (end 65.8421 57.4165) (width 0.5) (layer "F.Cu") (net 7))
 (via (at 69.5 76) (size 0.6) (drill 0.3) (layers "F.Cu" "B.Cu") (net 7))
 (via (at 77.0921 69.4165) (size 0.6) (drill 0.3) (layers "F.Cu" "B.Cu") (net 7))
 (segment (start 81 70) (end 80 70) (width 0.5) (layer "B.Cu") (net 7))
 (segment (start 81 76) (end 81 70) (width 0.5) (layer "B.Cu") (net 7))
 (segment (start 69.5 76) (end 81 76) (width 0.5) (layer "B.Cu") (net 7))
 (segment (start 79.4165 69.4165) (end 77.0921 69.4165) (width 0.5) (layer "B.Cu") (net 7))
 (segment (start 80 70) (end 79.4165 69.4165) (width 0.5) (layer "B.Cu") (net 7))
 (segment (start 86.4521 80.1165) (end 79.1521 72.8165) (width 0.5) (layer "F.Cu") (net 5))
 (segment (start 70.2756 66) (end 70.5 66) (width 0.2) (layer "F.Cu") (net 5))
 (segment (start 67.5921 82.3165) (end 65.0921 82.3165) (width 0.5) (layer "F.Cu") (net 5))
 (segment (start 79.1521 72.8165) (end 77.0921 72.8165) (width 0.5) (layer "F.Cu") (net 5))
 (segment (start 68.8165 60.8165) (end 70.2756 62.2756) (width 0.5) (layer "F.Cu") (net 5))
 (segment (start 77.0921 72.8165) (end 67.5921 82.3165) (width 0.5) (layer "F.Cu") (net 5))
 (segment (start 70.2756 62.2756) (end 70.2756 66) (width 0.5) (layer "F.Cu") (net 5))
 (segment (start 65.0921 60.8165) (end 68.8165 60.8165) (width 0.5) (layer "F.Cu") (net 5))
 (via (at 77.0921 72.8165) (size 0.6) (drill 0.3) (layers "F.Cu" "B.Cu") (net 5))
 (via (at 70.5 66) (size 0.6) (drill 0.3) (layers "F.Cu" "B.Cu") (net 5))
 (segment (start 77.0921 72.5921) (end 77.0921 72.8165) (width 0.2) (layer "B.Cu") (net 5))
 (segment (start 70.5 66) (end 77.0921 72.5921) (width 0.5) (layer "B.Cu") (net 5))
 (segment (start 65.0921 59.1165) (end 65.5 59.1165) (width 0.2) (layer "F.Cu") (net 6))
 (segment (start 76.6421 71.1165) (end 77.0921 71.1165) (width 0.2) (layer "F.Cu") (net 6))
 (segment (start 71.6165 59.1165) (end 65.5 59.1165) (width 0.5) (layer "F.Cu") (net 6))
 (segment (start 75.6165 71.1165) (end 75 70.5) (width 0.5) (layer "F.Cu") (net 6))
 (segment (start 66.8835 80.6165) (end 65.0921 80.6165) (width 0.5) (layer "F.Cu") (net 6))
 (segment (start 65.0921 59.1165) (end 65.9086 59.1165) (width 0.2) (layer "F.Cu") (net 6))
 (segment (start 76.3835 71.1165) (end 66.8835 80.6165) (width 0.5) (layer "F.Cu") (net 6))
 (segment (start 86.4521 72.1165) (end 85.4521 71.1165) (width 0.2) (layer "F.Cu") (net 6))
 (segment (start 75 62.5) (end 71.6165 59.1165) (width 0.5) (layer "F.Cu") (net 6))
 (segment (start 77.0921 71.1165) (end 76.3835 71.1165) (width 0.2) (layer "F.Cu") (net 6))
 (segment (start 75 70.5) (end 75 62.5) (width 0.5) (layer "F.Cu") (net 6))
 (segment (start 85.4521 71.1165) (end 77.0921 71.1165) (width 0.5) (layer "F.Cu") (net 6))
 (segment (start 76.3835 71.1165) (end 75.6165 71.1165) (width 0.5) (layer "F.Cu") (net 6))
 (via (at 115.214 72.1788) (size 0.6) (drill 0.3) (layers "F.Cu" "B.Cu") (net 9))
 (segment (start 112 91.46) (end 112 72.5) (width 0.5) (layer "B.Cu") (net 9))
 (segment (start 115.214 77.874) (end 116.5 79.16) (width 0.5) (layer "B.Cu") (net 9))
 (segment (start 114.8928 72.5) (end 115.214 72.1788) (width 0.2) (layer "B.Cu") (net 9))
 (segment (start 112 72.5) (end 114.8928 72.5) (width 0.5) (layer "B.Cu") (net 9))
 (segment (start 115.214 72.1788) (end 115.214 77.874) (width 0.5) (layer "B.Cu") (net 9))
 (segment (start 110 93.46) (end 112 91.46) (width 0.5) (layer "B.Cu") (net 9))
 (via (at 128.214 72.1788) (size 0.6) (drill 0.3) (layers "F.Cu" "B.Cu") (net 12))
 (segment (start 128.214 78.874) (end 128.5 79.16) (width 0.2) (layer "B.Cu") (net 12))
 (segment (start 128.214 72.1788) (end 128.214 78.874) (width 0.5) (layer "B.Cu") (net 12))
 (segment (start 124 82) (end 124 73) (width 0.5) (layer "B.Cu") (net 12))
 (segment (start 127.3928 73) (end 128.214 72.1788) (width 0.5) (layer "B.Cu") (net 12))
 (segment (start 112.54 93.46) (end 124 82) (width 0.5) (layer "B.Cu") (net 12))
 (segment (start 124 73) (end 127.3928 73) (width 0.5) (layer "B.Cu") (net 12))
 (segment (start 145.46 88.48) (end 140.48 93.46) (width 0.5) (layer "F.Cu") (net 13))
 (segment (start 145.46 85.5) (end 145.46 88.48) (width 0.5) (layer "F.Cu") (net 13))
 (segment (start 148 85.5) (end 134.6788 72.1788) (width 0.5) (layer "F.Cu") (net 2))
 (segment (start 134.6788 72.1788) (end 132.786 72.1788) (width 0.5) (layer "F.Cu") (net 2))
 (segment (start 132.786 74.214) (end 132 75) (width 0.5) (layer "F.Cu") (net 2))
 (segment (start 132 75) (end 120 75) (width 0.5) (layer "F.Cu") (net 2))
 (segment (start 149.25 86.75) (end 148 85.5) (width 0.4) (layer "F.Cu") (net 2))
 (segment (start 151 88.5) (end 151 96) (width 0.5) (layer "F.Cu") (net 2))
 (segment (start 132.786 72.1788) (end 132.786 74.214) (width 0.5) (layer "F.Cu") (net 2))
 (segment (start 106.286 74.286) (end 106.286 72.1788) (width 0.5) (layer "F.Cu") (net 2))
 (segment (start 119.786 72.1788) (end 119.786 74.786) (width 0.5) (layer "F.Cu") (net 2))
 (segment (start 151 96) (end 148.1 96) (width 0.5) (layer "F.Cu") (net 2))
 (segment (start 149.25 86.75) (end 151 88.5) (width 0.5) (layer "F.Cu") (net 2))
 (segment (start 120 75) (end 107 75) (width 0.5) (layer "F.Cu") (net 2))
 (segment (start 107 75) (end 106.286 74.286) (width 0.5) (layer "F.Cu") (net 2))
 (segment (start 119.786 74.786) (end 120 75) (width 0.2) (layer "F.Cu") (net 2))
 (via (at 101.714 72.1788) (size 0.6) (drill 0.3) (layers "F.Cu" "B.Cu") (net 1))
 (segment (start 101.714 87.714) (end 101.714 72.1788) (width 0.5) (layer "B.Cu") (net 1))
 (segment (start 101.714 72.1788) (end 101.714 74.874) (width 0.5) (layer "B.Cu") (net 1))
 (segment (start 107.46 93.46) (end 101.714 87.714) (width 0.5) (layer "B.Cu") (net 1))
 (segment (start 101.714 74.874) (end 106 79.16) (width 0.5) (layer "B.Cu") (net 1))
 (segment (start 142.92 85.5) (end 138.92 81.5) (width 0.5) (layer "F.Cu") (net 14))
 (segment (start 137 81.5) (end 137 86.78) (width 0.5) (layer "F.Cu") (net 14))
 (segment (start 138.92 81.5) (end 137 81.5) (width 0.5) (layer "F.Cu") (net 14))
 (segment (start 137 86.78) (end 130.32 93.46) (width 0.5) (layer "F.Cu") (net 14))
 (segment (start 106 84.24) (end 116.5 84.24) (width 0.5) (layer "F.Cu") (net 11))
 (segment (start 116.5 84.24) (end 128.5 84.24) (width 0.5) (layer "F.Cu") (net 11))
 (segment (start 131 89.5) (end 128.5 87) (width 0.5) (layer "B.Cu") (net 11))
 (segment (start 148.1 93.46) (end 146.95 92.31) (width 0.5) (layer "B.Cu") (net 11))
 (segment (start 128.5 87) (end 128.5 84.24) (width 0.5) (layer "B.Cu") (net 11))
 (segment (start 146.95 92.31) (end 146.95 89.95) (width 0.5) (layer "B.Cu") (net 11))
 (segment (start 146.95 89.95) (end 146.5 89.5) (width 0.5) (layer "B.Cu") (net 11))
 (segment (start 146.5 89.5) (end 131 89.5) (width 0.5) (layer "B.Cu") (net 11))
 (segment (start 95.8835 72.1165) (end 104 64) (width 0.5) (layer "F.Cu") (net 3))
 (segment (start 91.5321 72.1165) (end 95.8835 72.1165) (width 0.5) (layer "F.Cu") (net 3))
 (via (at 117.5 64) (size 0.6) (drill 0.3) (layers "F.Cu" "B.Cu") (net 10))
 (segment (start 99.5 59.5) (end 113 59.5) (width 0.5) (layer "B.Cu") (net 10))
 (segment (start 91.5321 76) (end 96.5 76) (width 0.5) (layer "B.Cu") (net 10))
 (segment (start 113 59.5) (end 117.5 64) (width 0.5) (layer "B.Cu") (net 10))
 (segment (start 91.5321 80.1165) (end 91.5321 76) (width 0.5) (layer "B.Cu") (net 10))
 (segment (start 96.5 76) (end 96.5 62.5) (width 0.5) (layer "B.Cu") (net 10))
 (segment (start 96.5 62.5) (end 99.5 59.5) (width 0.5) (layer "B.Cu") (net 10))
 (segment (start 127.5 57.5) (end 96 57.5) (width 0.5) (layer "F.Cu") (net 8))
 (segment (start 91.6921 61.8079) (end 91.6921 64.1165) (width 0.5) (layer "F.Cu") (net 8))
 (segment (start 96 57.5) (end 91.6921 61.8079) (width 0.5) (layer "F.Cu") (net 8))
 (segment (start 130.5 64) (end 130.5 60.5) (width 0.5) (layer "F.Cu") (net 8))
 (segment (start 130.5 60.5) (end 127.5 57.5) (width 0.5) (layer "F.Cu") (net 8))
 (segment (start 140.38 85.5) (end 137.94 87.94) (width 0.5) (layer "F.Cu") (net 15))
 (segment (start 137.94 87.94) (end 137.94 93.46) (width 0.5) (layer "F.Cu") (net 15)))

